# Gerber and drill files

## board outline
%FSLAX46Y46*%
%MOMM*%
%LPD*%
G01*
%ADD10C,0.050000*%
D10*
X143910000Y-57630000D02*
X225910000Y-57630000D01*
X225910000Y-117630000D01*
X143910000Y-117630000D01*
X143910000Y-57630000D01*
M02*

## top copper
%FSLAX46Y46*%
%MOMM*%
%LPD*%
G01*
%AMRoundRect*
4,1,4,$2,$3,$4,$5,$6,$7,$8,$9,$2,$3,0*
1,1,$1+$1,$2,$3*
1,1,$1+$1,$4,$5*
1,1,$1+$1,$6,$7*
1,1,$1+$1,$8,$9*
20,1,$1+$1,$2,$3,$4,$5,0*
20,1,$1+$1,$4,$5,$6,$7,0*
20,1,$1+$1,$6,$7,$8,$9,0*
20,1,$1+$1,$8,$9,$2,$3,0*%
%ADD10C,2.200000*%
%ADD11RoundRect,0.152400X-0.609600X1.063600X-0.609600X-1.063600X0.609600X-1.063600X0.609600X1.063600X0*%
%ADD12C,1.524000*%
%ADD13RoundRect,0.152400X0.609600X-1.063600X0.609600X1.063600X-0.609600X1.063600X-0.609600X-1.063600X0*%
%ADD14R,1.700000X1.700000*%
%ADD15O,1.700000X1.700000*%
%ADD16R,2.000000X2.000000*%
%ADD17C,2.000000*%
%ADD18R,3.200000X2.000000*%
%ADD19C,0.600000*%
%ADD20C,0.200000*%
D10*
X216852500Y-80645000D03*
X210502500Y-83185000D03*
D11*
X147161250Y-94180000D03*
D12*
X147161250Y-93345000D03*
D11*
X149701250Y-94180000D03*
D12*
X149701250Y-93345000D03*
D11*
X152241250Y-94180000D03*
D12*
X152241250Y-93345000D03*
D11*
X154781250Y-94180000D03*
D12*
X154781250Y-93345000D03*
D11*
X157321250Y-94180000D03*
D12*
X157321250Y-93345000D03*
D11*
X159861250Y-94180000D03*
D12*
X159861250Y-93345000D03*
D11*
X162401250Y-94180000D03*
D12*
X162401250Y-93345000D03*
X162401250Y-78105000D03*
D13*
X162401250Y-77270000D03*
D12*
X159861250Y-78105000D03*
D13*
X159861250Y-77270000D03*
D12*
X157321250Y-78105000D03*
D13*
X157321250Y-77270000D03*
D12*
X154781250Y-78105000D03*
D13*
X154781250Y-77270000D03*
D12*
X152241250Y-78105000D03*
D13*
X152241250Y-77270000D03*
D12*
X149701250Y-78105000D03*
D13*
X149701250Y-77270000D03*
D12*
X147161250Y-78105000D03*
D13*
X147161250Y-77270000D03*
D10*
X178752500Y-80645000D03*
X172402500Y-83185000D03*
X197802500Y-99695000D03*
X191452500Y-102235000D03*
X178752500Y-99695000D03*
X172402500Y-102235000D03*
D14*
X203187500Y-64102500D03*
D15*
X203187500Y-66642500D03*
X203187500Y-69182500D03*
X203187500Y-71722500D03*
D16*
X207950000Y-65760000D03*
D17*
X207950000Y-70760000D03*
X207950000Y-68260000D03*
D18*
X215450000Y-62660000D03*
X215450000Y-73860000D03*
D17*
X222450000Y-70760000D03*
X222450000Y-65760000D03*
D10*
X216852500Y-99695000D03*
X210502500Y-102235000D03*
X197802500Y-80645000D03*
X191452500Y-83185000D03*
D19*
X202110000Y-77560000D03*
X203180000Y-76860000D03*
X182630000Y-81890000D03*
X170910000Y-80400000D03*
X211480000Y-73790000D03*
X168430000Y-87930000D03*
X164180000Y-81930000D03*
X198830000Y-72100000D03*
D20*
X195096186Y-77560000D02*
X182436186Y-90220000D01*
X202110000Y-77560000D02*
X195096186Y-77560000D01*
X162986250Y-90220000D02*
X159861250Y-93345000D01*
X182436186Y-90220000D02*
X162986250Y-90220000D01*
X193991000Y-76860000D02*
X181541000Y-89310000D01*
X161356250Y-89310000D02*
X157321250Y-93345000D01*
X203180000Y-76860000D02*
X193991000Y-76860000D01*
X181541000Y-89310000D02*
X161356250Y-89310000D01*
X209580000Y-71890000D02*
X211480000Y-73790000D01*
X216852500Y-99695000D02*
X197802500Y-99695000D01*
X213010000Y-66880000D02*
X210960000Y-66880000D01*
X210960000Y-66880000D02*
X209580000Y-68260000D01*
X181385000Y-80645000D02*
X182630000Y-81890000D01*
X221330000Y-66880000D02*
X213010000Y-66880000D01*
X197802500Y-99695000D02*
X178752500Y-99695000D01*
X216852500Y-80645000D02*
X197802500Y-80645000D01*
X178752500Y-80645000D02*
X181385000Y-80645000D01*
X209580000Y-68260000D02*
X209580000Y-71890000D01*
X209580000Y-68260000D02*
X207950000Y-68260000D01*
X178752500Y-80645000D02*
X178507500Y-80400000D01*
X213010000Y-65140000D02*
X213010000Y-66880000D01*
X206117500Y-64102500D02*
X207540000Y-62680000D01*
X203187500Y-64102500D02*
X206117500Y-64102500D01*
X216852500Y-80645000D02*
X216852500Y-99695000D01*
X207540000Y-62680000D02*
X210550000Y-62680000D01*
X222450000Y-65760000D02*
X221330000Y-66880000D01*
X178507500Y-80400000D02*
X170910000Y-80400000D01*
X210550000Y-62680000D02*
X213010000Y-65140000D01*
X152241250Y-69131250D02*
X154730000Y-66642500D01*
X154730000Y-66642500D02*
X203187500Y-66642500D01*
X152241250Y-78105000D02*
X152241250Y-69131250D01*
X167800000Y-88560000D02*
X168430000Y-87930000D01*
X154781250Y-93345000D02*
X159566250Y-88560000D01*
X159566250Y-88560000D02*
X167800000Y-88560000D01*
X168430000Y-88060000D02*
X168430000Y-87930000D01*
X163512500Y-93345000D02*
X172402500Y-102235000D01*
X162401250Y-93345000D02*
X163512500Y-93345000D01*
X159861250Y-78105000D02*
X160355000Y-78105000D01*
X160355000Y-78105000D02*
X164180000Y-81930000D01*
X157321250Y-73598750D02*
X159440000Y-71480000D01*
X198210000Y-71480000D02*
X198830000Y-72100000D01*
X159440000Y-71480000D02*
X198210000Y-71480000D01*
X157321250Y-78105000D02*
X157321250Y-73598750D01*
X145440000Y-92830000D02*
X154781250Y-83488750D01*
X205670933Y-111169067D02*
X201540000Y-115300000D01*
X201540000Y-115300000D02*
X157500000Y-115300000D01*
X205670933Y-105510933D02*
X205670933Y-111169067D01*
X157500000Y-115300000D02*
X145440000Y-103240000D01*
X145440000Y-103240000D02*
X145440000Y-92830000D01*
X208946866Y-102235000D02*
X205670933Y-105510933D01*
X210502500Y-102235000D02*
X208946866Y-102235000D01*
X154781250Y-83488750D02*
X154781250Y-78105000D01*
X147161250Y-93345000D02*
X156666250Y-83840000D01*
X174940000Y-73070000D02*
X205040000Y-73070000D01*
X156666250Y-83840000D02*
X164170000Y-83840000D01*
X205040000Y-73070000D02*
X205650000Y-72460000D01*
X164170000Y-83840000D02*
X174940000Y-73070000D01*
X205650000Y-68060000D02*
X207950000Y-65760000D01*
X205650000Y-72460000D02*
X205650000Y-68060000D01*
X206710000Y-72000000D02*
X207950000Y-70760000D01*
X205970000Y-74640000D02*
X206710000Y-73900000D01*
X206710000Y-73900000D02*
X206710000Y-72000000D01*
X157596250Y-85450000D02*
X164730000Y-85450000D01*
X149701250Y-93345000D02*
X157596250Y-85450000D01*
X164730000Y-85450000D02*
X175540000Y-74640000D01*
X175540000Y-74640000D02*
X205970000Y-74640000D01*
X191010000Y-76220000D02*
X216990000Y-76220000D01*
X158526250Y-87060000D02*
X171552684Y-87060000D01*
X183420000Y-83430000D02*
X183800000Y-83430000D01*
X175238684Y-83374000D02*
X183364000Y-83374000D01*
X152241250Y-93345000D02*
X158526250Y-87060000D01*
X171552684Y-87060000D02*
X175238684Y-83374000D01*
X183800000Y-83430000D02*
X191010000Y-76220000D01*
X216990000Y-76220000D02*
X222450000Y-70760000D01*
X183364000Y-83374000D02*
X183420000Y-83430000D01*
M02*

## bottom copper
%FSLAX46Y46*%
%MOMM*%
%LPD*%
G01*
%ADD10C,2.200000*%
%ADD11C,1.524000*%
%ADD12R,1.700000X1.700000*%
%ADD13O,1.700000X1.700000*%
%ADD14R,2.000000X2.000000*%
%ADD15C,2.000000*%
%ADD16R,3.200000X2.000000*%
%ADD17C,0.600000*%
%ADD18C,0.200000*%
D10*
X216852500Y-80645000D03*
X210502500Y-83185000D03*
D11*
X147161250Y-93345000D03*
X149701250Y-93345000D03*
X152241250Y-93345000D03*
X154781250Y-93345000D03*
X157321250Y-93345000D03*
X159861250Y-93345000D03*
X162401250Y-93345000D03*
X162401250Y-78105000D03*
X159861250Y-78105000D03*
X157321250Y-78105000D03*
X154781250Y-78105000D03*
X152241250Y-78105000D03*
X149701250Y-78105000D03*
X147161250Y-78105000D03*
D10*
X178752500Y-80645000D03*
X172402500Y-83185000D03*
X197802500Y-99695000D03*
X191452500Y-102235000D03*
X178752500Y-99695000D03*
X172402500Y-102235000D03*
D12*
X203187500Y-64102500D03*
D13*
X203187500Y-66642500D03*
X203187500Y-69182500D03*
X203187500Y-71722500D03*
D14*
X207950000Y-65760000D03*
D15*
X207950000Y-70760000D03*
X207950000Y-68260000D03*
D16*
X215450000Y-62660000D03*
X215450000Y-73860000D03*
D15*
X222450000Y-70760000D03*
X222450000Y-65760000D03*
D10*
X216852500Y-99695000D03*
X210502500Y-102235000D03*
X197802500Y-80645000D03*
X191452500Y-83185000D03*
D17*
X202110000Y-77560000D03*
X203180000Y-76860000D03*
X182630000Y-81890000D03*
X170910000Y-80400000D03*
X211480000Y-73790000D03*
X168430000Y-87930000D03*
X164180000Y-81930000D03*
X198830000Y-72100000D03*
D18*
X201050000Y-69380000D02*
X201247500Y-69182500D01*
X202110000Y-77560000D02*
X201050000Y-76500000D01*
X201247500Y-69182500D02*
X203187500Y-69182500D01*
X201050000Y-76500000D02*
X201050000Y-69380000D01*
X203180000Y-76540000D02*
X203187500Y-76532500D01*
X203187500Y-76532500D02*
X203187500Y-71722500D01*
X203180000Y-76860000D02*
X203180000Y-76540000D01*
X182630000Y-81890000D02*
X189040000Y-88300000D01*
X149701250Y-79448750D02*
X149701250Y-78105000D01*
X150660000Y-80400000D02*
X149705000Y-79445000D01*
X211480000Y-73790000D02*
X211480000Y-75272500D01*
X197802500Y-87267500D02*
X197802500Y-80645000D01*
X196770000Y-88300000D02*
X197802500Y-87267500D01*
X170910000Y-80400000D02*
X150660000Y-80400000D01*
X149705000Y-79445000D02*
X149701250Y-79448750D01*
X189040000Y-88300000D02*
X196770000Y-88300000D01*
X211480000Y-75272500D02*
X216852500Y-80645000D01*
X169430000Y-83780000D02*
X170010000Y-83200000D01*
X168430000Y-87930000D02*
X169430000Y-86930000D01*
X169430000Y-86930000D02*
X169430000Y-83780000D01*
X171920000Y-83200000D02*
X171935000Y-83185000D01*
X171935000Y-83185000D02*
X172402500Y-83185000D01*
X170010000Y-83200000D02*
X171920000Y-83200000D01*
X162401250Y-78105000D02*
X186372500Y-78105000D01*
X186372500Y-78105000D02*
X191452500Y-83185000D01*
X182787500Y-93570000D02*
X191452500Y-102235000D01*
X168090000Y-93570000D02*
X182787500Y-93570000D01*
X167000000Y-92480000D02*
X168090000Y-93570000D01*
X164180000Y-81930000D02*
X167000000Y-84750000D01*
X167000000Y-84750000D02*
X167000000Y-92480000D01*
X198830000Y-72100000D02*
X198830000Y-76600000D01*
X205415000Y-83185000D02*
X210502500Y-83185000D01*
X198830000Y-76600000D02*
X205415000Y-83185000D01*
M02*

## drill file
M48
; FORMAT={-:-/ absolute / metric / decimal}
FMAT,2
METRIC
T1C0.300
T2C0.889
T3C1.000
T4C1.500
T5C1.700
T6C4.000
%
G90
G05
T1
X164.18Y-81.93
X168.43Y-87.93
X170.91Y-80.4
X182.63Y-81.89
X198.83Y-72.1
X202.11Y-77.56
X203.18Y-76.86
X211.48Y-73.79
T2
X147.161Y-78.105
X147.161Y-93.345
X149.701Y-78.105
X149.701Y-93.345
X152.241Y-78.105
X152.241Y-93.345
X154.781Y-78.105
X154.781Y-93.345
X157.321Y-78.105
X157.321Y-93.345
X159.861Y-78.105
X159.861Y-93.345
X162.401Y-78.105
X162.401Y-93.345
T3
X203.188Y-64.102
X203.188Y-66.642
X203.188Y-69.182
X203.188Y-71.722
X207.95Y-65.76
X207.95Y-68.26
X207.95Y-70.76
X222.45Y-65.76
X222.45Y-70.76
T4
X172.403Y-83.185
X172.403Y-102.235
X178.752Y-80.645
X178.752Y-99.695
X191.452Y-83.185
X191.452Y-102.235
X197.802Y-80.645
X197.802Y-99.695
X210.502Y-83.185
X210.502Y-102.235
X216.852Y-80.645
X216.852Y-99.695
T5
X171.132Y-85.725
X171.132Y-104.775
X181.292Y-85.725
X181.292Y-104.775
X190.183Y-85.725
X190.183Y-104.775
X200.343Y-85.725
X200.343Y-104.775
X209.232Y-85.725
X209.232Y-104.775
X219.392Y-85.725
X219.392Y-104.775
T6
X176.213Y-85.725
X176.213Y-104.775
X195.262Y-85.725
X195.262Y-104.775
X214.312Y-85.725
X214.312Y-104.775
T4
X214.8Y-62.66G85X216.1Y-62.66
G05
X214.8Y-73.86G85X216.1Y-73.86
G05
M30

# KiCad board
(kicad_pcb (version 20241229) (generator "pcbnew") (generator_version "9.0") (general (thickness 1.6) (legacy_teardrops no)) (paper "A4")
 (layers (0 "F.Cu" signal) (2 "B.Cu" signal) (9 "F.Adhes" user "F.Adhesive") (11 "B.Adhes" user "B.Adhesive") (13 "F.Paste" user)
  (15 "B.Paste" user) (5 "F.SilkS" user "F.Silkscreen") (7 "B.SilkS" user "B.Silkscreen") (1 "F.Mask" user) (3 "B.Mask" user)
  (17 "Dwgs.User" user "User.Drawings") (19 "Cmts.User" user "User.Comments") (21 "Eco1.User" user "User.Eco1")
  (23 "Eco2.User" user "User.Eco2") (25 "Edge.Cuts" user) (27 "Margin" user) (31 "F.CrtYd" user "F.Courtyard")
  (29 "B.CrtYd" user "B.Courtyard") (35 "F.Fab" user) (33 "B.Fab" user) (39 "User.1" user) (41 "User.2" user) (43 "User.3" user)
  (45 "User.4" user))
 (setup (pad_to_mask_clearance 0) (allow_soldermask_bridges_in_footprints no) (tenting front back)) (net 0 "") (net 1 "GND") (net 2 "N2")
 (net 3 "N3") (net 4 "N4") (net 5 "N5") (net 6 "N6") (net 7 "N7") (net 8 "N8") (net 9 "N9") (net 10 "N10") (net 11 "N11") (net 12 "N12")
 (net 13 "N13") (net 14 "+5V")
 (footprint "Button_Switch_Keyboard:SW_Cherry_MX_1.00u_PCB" (layer "F.Cu") (at 216.8525 80.645)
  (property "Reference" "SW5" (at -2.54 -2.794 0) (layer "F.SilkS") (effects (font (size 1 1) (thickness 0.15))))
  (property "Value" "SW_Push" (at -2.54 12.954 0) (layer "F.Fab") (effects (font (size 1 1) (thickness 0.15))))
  (pad "" np_thru_hole circle (at -7.62 5.08) (size 1.7 1.7) (drill 1.7) (layers "*.Cu" "*.Mask"))
  (pad "" np_thru_hole circle (at -2.54 5.08) (size 4 4) (drill 4) (layers "*.Cu" "*.Mask"))
  (pad "" np_thru_hole circle (at 2.54 5.08) (size 1.7 1.7) (drill 1.7) (layers "*.Cu" "*.Mask"))
  (pad "1" thru_hole circle (at 0 0) (size 2.2 2.2) (drill 1.5) (layers "*.Cu" "*.Mask") (remove_unused_layers no) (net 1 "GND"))
  (pad "2" thru_hole circle (at -6.35 2.54) (size 2.2 2.2) (drill 1.5) (layers "*.Cu" "*.Mask") (remove_unused_layers no) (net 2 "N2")))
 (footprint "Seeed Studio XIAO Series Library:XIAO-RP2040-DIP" (layer "F.Cu") (at 154.78125 85.725 90)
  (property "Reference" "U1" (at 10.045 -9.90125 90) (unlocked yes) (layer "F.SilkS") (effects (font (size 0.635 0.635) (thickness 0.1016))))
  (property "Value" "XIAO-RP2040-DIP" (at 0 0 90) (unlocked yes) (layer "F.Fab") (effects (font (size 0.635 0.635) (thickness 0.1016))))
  (pad "1" smd roundrect (at -8.455 -7.62 270) (size 2.432 1.524) (layers "F.Cu" "F.Mask") (roundrect_rratio 0.1) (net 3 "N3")
   (thermal_bridge_angle 45))
  (pad "1" thru_hole circle (at -7.62 -7.62 270) (size 1.524 1.524) (drill 0.889) (layers "*.Cu" "*.Mask") (remove_unused_layers no)
   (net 3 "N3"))
  (pad "2" smd roundrect (at -8.455 -5.08 270) (size 2.432 1.524) (layers "F.Cu" "F.Mask") (roundrect_rratio 0.1) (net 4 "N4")
   (thermal_bridge_angle 45))
  (pad "2" thru_hole circle (at -7.62 -5.08 270) (size 1.524 1.524) (drill 0.889) (layers "*.Cu" "*.Mask") (remove_unused_layers no)
   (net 4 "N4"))
  (pad "3" smd roundrect (at -8.455 -2.54 270) (size 2.432 1.524) (layers "F.Cu" "F.Mask") (roundrect_rratio 0.1) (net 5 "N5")
   (thermal_bridge_angle 45))
  (pad "3" thru_hole circle (at -7.62 -2.54 270) (size 1.524 1.524) (drill 0.889) (layers "*.Cu" "*.Mask") (remove_unused_layers no)
   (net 5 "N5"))
  (pad "4" smd roundrect (at -8.455 0 270) (size 2.432 1.524) (layers "F.Cu" "F.Mask") (roundrect_rratio 0.1) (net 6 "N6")
   (thermal_bridge_angle 45))
  (pad "4" thru_hole circle (at -7.62 0 270) (size 1.524 1.524) (drill 0.889) (layers "*.Cu" "*.Mask") (remove_unused_layers no)
   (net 6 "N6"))
  (pad "5" smd roundrect (at -8.455 2.54 270) (size 2.432 1.524) (layers "F.Cu" "F.Mask") (roundrect_rratio 0.1) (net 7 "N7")
   (thermal_bridge_angle 45))
  (pad "5" thru_hole circle (at -7.62 2.54 270) (size 1.524 1.524) (drill 0.889) (layers "*.Cu" "*.Mask") (remove_unused_layers no)
   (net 7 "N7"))
  (pad "6" smd roundrect (at -8.455 5.08 270) (size 2.432 1.524) (layers "F.Cu" "F.Mask") (roundrect_rratio 0.1) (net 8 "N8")
   (thermal_bridge_angle 45))
  (pad "6" thru_hole circle (at -7.62 5.08 270) (size 1.524 1.524) (drill 0.889) (layers "*.Cu" "*.Mask") (remove_unused_layers no)
   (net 8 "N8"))
  (pad "7" smd roundrect (at -8.455 7.62 270) (size 2.432 1.524) (layers "F.Cu" "F.Mask") (roundrect_rratio 0.1) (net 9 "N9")
   (thermal_bridge_angle 45))
  (pad "7" thru_hole circle (at -7.62 7.62 270) (size 1.524 1.524) (drill 0.889) (layers "*.Cu" "*.Mask") (remove_unused_layers no)
   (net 9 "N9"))
  (pad "8" thru_hole circle (at 7.62 7.62 90) (size 1.524 1.524) (drill 0.889) (layers "*.Cu" "*.Mask") (remove_unused_layers no)
   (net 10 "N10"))
  (pad "8" smd roundrect (at 8.455 7.62 90) (size 2.432 1.524) (layers "F.Cu" "F.Mask") (roundrect_rratio 0.1) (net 10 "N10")
   (thermal_bridge_angle 45))
  (pad "9" thru_hole circle (at 7.62 5.08 90) (size 1.524 1.524) (drill 0.889) (layers "*.Cu" "*.Mask") (remove_unused_layers no)
   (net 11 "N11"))
  (pad "9" smd roundrect (at 8.455 5.08 90) (size 2.432 1.524) (layers "F.Cu" "F.Mask") (roundrect_rratio 0.1) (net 11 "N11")
   (thermal_bridge_angle 45))
  (pad "10" thru_hole circle (at 7.62 2.54 90) (size 1.524 1.524) (drill 0.889) (layers "*.Cu" "*.Mask") (remove_unused_layers no)
   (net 2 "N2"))
  (pad "10" smd roundrect (at 8.455 2.54 90) (size 2.432 1.524) (layers "F.Cu" "F.Mask") (roundrect_rratio 0.1) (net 2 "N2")
   (thermal_bridge_angle 45))
  (pad "11" thru_hole circle (at 7.62 0 90) (size 1.524 1.524) (drill 0.889) (layers "*.Cu" "*.Mask") (remove_unused_layers no)
   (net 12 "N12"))
  (pad "11" smd roundrect (at 8.455 0 90) (size 2.432 1.524) (layers "F.Cu" "F.Mask") (roundrect_rratio 0.1) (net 12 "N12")
   (thermal_bridge_angle 45))
  (pad "12" thru_hole circle (at 7.62 -2.54 90) (size 1.524 1.524) (drill 0.889) (layers "*.Cu" "*.Mask") (remove_unused_layers no)
   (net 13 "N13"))
  (pad "12" smd roundrect (at 8.455 -2.54 90) (size 2.432 1.524) (layers "F.Cu" "F.Mask") (roundrect_rratio 0.1) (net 13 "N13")
   (thermal_bridge_angle 45))
  (pad "13" thru_hole circle (at 7.62 -5.08 90) (size 1.524 1.524) (drill 0.889) (layers "*.Cu" "*.Mask") (remove_unused_layers no)
   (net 1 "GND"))
  (pad "13" smd roundrect (at 8.455 -5.08 90) (size 2.432 1.524) (layers "F.Cu" "F.Mask") (roundrect_rratio 0.1) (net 1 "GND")
   (thermal_bridge_angle 45))
  (pad "14" thru_hole circle (at 7.62 -7.62 90) (size 1.524 1.524) (drill 0.889) (layers "*.Cu" "*.Mask") (remove_unused_layers no)
   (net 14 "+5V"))
  (pad "14" smd roundrect (at 8.455 -7.62 90) (size 2.432 1.524) (layers "F.Cu" "F.Mask") (roundrect_rratio 0.1) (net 14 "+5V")
   (thermal_bridge_angle 45)))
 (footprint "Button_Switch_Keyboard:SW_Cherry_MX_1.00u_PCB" (layer "F.Cu") (at 178.7525 80.645)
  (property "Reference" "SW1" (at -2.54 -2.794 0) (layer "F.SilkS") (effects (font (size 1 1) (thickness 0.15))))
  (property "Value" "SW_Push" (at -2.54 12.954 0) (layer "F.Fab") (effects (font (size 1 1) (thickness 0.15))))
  (pad "" np_thru_hole circle (at -7.62 5.08) (size 1.7 1.7) (drill 1.7) (layers "*.Cu" "*.Mask"))
  (pad "" np_thru_hole circle (at -2.54 5.08) (size 4 4) (drill 4) (layers "*.Cu" "*.Mask"))
  (pad "" np_thru_hole circle (at 2.54 5.08) (size 1.7 1.7) (drill 1.7) (layers "*.Cu" "*.Mask"))
  (pad "1" thru_hole circle (at 0 0) (size 2.2 2.2) (drill 1.5) (layers "*.Cu" "*.Mask") (remove_unused_layers no) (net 1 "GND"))
  (pad "2" thru_hole circle (at -6.35 2.54) (size 2.2 2.2) (drill 1.5) (layers "*.Cu" "*.Mask") (remove_unused_layers no) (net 6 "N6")))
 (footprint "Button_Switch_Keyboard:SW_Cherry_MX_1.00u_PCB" (layer "F.Cu") (at 197.8025 99.695)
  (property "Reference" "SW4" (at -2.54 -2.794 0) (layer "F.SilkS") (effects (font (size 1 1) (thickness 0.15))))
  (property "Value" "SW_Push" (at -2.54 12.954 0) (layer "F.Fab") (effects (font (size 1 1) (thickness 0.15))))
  (pad "" np_thru_hole circle (at -7.62 5.08) (size 1.7 1.7) (drill 1.7) (layers "*.Cu" "*.Mask"))
  (pad "" np_thru_hole circle (at -2.54 5.08) (size 4 4) (drill 4) (layers "*.Cu" "*.Mask"))
  (pad "" np_thru_hole circle (at 2.54 5.08) (size 1.7 1.7) (drill 1.7) (layers "*.Cu" "*.Mask"))
  (pad "1" thru_hole circle (at 0 0) (size 2.2 2.2) (drill 1.5) (layers "*.Cu" "*.Mask") (remove_unused_layers no) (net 1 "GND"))
  (pad "2" thru_hole circle (at -6.35 2.54) (size 2.2 2.2) (drill 1.5) (layers "*.Cu" "*.Mask") (remove_unused_layers no) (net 11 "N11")))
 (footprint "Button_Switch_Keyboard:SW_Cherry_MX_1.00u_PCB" (layer "F.Cu") (at 178.7525 99.695)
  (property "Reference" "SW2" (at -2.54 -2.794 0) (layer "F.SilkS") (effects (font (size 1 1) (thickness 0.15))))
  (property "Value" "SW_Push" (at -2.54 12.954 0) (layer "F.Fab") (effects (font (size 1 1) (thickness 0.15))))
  (pad "" np_thru_hole circle (at -7.62 5.08) (size 1.7 1.7) (drill 1.7) (layers "*.Cu" "*.Mask"))
  (pad "" np_thru_hole circle (at -2.54 5.08) (size 4 4) (drill 4) (layers "*.Cu" "*.Mask"))
  (pad "" np_thru_hole circle (at 2.54 5.08) (size 1.7 1.7) (drill 1.7) (layers "*.Cu" "*.Mask"))
  (pad "1" thru_hole circle (at 0 0) (size 2.2 2.2) (drill 1.5) (layers "*.Cu" "*.Mask") (remove_unused_layers no) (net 1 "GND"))
  (pad "2" thru_hole circle (at -6.35 2.54) (size 2.2 2.2) (drill 1.5) (layers "*.Cu" "*.Mask") (remove_unused_layers no) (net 9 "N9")))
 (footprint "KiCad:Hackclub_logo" (layer "F.Cu") (at 156.223071 67.360382)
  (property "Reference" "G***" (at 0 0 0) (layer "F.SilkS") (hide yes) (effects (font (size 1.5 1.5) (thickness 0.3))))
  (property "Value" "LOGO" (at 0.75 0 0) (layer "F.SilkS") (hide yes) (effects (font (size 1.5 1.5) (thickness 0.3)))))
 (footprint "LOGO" (layer "F.Cu") (at 155.84 108.43)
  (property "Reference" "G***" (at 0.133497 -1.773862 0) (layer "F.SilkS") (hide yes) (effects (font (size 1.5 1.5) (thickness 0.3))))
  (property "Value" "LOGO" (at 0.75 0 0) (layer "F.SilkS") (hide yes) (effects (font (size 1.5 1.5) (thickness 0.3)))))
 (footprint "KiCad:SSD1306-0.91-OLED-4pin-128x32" (layer "F.Cu") (at 166.6875 61.9125)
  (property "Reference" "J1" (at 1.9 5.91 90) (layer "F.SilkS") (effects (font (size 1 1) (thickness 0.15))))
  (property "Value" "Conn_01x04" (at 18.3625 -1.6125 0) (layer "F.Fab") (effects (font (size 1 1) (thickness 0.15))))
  (pad "1" thru_hole rect (at 36.5 2.19) (size 1.7 1.7) (drill 1) (layers "*.Cu" "*.Mask") (remove_unused_layers no) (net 1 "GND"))
  (pad "2" thru_hole oval (at 36.5 4.73) (size 1.7 1.7) (drill 1) (layers "*.Cu" "*.Mask") (remove_unused_layers no) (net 13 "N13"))
  (pad "3" thru_hole oval (at 36.5 7.27) (size 1.7 1.7) (drill 1) (layers "*.Cu" "*.Mask") (remove_unused_layers no) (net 8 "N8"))
  (pad "4" thru_hole oval (at 36.5 9.81) (size 1.7 1.7) (drill 1) (layers "*.Cu" "*.Mask") (remove_unused_layers no) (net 7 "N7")))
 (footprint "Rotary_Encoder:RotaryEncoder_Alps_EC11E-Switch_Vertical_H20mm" (layer "F.Cu") (at 207.95 65.76)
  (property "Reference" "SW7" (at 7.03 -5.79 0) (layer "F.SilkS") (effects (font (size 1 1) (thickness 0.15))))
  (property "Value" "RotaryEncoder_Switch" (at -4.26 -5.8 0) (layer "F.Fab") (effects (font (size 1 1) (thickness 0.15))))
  (pad "A" thru_hole rect (at 0 0) (size 2 2) (drill 1) (layers "*.Cu" "*.Mask") (remove_unused_layers no) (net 3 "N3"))
  (pad "B" thru_hole circle (at 0 5) (size 2 2) (drill 1) (layers "*.Cu" "*.Mask") (remove_unused_layers no) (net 4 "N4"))
  (pad "C" thru_hole circle (at 0 2.5) (size 2 2) (drill 1) (layers "*.Cu" "*.Mask") (remove_unused_layers no) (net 1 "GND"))
  (pad "MP" thru_hole rect (at 7.5 -3.1) (size 3.2 2) (drill oval 2.8 1.5) (layers "*.Cu" "*.Mask") (remove_unused_layers no))
  (pad "MP" thru_hole rect (at 7.5 8.1) (size 3.2 2) (drill oval 2.8 1.5) (layers "*.Cu" "*.Mask") (remove_unused_layers no))
  (pad "S1" thru_hole circle (at 14.5 5) (size 2 2) (drill 1) (layers "*.Cu" "*.Mask") (remove_unused_layers no) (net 5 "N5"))
  (pad "S2" thru_hole circle (at 14.5 0) (size 2 2) (drill 1) (layers "*.Cu" "*.Mask") (remove_unused_layers no) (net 1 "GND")))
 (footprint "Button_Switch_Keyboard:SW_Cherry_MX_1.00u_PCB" (layer "F.Cu") (at 216.8525 99.695)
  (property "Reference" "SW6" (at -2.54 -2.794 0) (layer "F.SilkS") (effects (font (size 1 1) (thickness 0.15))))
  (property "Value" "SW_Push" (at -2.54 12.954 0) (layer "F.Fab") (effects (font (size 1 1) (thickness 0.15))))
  (pad "" np_thru_hole circle (at -7.62 5.08) (size 1.7 1.7) (drill 1.7) (layers "*.Cu" "*.Mask"))
  (pad "" np_thru_hole circle (at -2.54 5.08) (size 4 4) (drill 4) (layers "*.Cu" "*.Mask"))
  (pad "" np_thru_hole circle (at 2.54 5.08) (size 1.7 1.7) (drill 1.7) (layers "*.Cu" "*.Mask"))
  (pad "1" thru_hole circle (at 0 0) (size 2.2 2.2) (drill 1.5) (layers "*.Cu" "*.Mask") (remove_unused_layers no) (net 1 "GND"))
  (pad "2" thru_hole circle (at -6.35 2.54) (size 2.2 2.2) (drill 1.5) (layers "*.Cu" "*.Mask") (remove_unused_layers no) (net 12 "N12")))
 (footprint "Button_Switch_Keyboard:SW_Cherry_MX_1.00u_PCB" (layer "F.Cu") (at 197.8025 80.645)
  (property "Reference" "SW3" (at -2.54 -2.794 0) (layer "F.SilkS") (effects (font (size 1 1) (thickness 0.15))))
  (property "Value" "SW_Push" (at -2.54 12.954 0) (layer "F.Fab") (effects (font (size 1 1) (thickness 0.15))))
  (pad "" np_thru_hole circle (at -7.62 5.08) (size 1.7 1.7) (drill 1.7) (layers "*.Cu" "*.Mask"))
  (pad "" np_thru_hole circle (at -2.54 5.08) (size 4 4) (drill 4) (layers "*.Cu" "*.Mask"))
  (pad "" np_thru_hole circle (at 2.54 5.08) (size 1.7 1.7) (drill 1.7) (layers "*.Cu" "*.Mask"))
  (pad "1" thru_hole circle (at 0 0) (size 2.2 2.2) (drill 1.5) (layers "*.Cu" "*.Mask") (remove_unused_layers no) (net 1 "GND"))
  (pad "2" thru_hole circle (at -6.35 2.54) (size 2.2 2.2) (drill 1.5) (layers "*.Cu" "*.Mask") (remove_unused_layers no) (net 10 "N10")))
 (gr_rect (start 143.91 57.63) (end 225.91 117.63) (stroke (width 0.05) (type solid)) (fill no) (layer "Edge.Cuts"))
 (segment (start 195.096186 77.56) (end 182.436186 90.22) (width 0.2) (layer "F.Cu") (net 8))
 (segment (start 202.11 77.56) (end 195.096186 77.56) (width 0.2) (layer "F.Cu") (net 8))
 (segment (start 162.98625 90.22) (end 159.86125 93.345) (width 0.2) (layer "F.Cu") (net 8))
 (segment (start 182.436186 90.22) (end 162.98625 90.22) (width 0.2) (layer "F.Cu") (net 8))
 (via (at 202.11 77.56) (size 0.6) (drill 0.3) (layers "F.Cu" "B.Cu") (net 8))
 (segment (start 201.05 69.38) (end 201.2475 69.1825) (width 0.2) (layer "B.Cu") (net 8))
 (segment (start 202.11 77.56) (end 201.05 76.5) (width 0.2) (layer "B.Cu") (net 8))
 (segment (start 201.2475 69.1825) (end 203.1875 69.1825) (width 0.2) (layer "B.Cu") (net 8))
 (segment (start 201.05 76.5) (end 201.05 69.38) (width 0.2) (layer "B.Cu") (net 8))
 (segment (start 193.991 76.86) (end 181.541 89.31) (width 0.2) (layer "F.Cu") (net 7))
 (segment (start 161.35625 89.31) (end 157.32125 93.345) (width 0.2) (layer "F.Cu") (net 7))
 (segment (start 203.18 76.86) (end 193.991 76.86) (width 0.2) (layer "F.Cu") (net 7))
 (segment (start 181.541 89.31) (end 161.35625 89.31) (width 0.2) (layer "F.Cu") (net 7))
 (via (at 203.18 76.86) (size 0.6) (drill 0.3) (layers "F.Cu" "B.Cu") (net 7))
 (segment (start 203.18 76.54) (end 203.1875 76.5325) (width 0.2) (layer "B.Cu") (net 7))
 (segment (start 203.1875 76.5325) (end 203.1875 71.7225) (width 0.2) (layer "B.Cu") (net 7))
 (segment (start 203.18 76.86) (end 203.18 76.54) (width 0.2) (layer "B.Cu") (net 7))
 (segment (start 209.58 71.89) (end 211.48 73.79) (width 0.2) (layer "F.Cu") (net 1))
 (segment (start 216.8525 99.695) (end 197.8025 99.695) (width 0.2) (layer "F.Cu") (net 1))
 (segment (start 213.01 66.88) (end 210.96 66.88) (width 0.2) (layer "F.Cu") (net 1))
 (segment (start 210.96 66.88) (end 209.58 68.26) (width 0.2) (layer "F.Cu") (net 1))
 (segment (start 181.385 80.645) (end 182.63 81.89) (width 0.2) (layer "F.Cu") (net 1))
 (segment (start 221.33 66.88) (end 213.01 66.88) (width 0.2) (layer "F.Cu") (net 1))
 (segment (start 197.8025 99.695) (end 178.7525 99.695) (width 0.2) (layer "F.Cu") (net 1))
 (segment (start 216.8525 80.645) (end 197.8025 80.645) (width 0.2) (layer "F.Cu") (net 1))
 (segment (start 178.7525 80.645) (end 181.385 80.645) (width 0.2) (layer "F.Cu") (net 1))
 (segment (start 209.58 68.26) (end 209.58 71.89) (width 0.2) (layer "F.Cu") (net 1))
 (segment (start 209.58 68.26) (end 207.95 68.26) (width 0.2) (layer "F.Cu") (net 1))
 (segment (start 178.7525 80.645) (end 178.5075 80.4) (width 0.2) (layer "F.Cu") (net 1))
 (segment (start 213.01 65.14) (end 213.01 66.88) (width 0.2) (layer "F.Cu") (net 1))
 (segment (start 206.1175 64.1025) (end 207.54 62.68) (width 0.2) (layer "F.Cu") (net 1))
 (segment (start 203.1875 64.1025) (end 206.1175 64.1025) (width 0.2) (layer "F.Cu") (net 1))
 (segment (start 216.8525 80.645) (end 216.8525 99.695) (width 0.2) (layer "F.Cu") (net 1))
 (segment (start 207.54 62.68) (end 210.55 62.68) (width 0.2) (layer "F.Cu") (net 1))
 (segment (start 222.45 65.76) (end 221.33 66.88) (width 0.2) (layer "F.Cu") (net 1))
 (segment (start 178.5075 80.4) (end 170.91 80.4) (width 0.2) (layer "F.Cu") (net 1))
 (segment (start 210.55 62.68) (end 213.01 65.14) (width 0.2) (layer "F.Cu") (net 1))
 (via (at 182.63 81.89) (size 0.6) (drill 0.3) (layers "F.Cu" "B.Cu") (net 1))
 (via (at 170.91 80.4) (size 0.6) (drill 0.3) (layers "F.Cu" "B.Cu") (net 1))
 (via (at 211.48 73.79) (size 0.6) (drill 0.3) (layers "F.Cu" "B.Cu") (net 1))
 (segment (start 182.63 81.89) (end 189.04 88.3) (width 0.2) (layer "B.Cu") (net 1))
 (segment (start 149.70125 79.44875) (end 149.70125 78.105) (width 0.2) (layer "B.Cu") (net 1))
 (segment (start 150.66 80.4) (end 149.705 79.445) (width 0.2) (layer "B.Cu") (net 1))
 (segment (start 211.48 73.79) (end 211.48 75.2725) (width 0.2) (layer "B.Cu") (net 1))
 (segment (start 197.8025 87.2675) (end 197.8025 80.645) (width 0.2) (layer "B.Cu") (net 1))
 (segment (start 196.77 88.3) (end 197.8025 87.2675) (width 0.2) (layer "B.Cu") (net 1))
 (segment (start 170.91 80.4) (end 150.66 80.4) (width 0.2) (layer "B.Cu") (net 1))
 (segment (start 149.705 79.445) (end 149.70125 79.44875) (width 0.2) (layer "B.Cu") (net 1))
 (segment (start 189.04 88.3) (end 196.77 88.3) (width 0.2) (layer "B.Cu") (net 1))
 (segment (start 211.48 75.2725) (end 216.8525 80.645) (width 0.2) (layer "B.Cu") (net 1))
 (segment (start 152.24125 69.13125) (end 154.73 66.6425) (width 0.2) (layer "F.Cu") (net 13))
 (segment (start 154.73 66.6425) (end 203.1875 66.6425) (width 0.2) (layer "F.Cu") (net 13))
 (segment (start 152.24125 78.105) (end 152.24125 69.13125) (width 0.2) (layer "F.Cu") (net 13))
 (segment (start 167.8 88.56) (end 168.43 87.93) (width 0.2) (layer "F.Cu") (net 6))
 (segment (start 154.78125 93.345) (end 159.56625 88.56) (width 0.2) (layer "F.Cu") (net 6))
 (segment (start 159.56625 88.56) (end 167.8 88.56) (width 0.2) (layer "F.Cu") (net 6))
 (segment (start 168.43 88.06) (end 168.43 87.93) (width 0.2) (layer "F.Cu") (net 6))
 (via (at 168.43 87.93) (size 0.6) (drill 0.3) (layers "F.Cu" "B.Cu") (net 6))
 (segment (start 169.43 83.78) (end 170.01 83.2) (width 0.2) (layer "B.Cu") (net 6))
 (segment (start 168.43 87.93) (end 169.43 86.93) (width 0.2) (layer "B.Cu") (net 6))
 (segment (start 169.43 86.93) (end 169.43 83.78) (width 0.2) (layer "B.Cu") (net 6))
 (segment (start 171.92 83.2) (end 171.935 83.185) (width 0.2) (layer "B.Cu") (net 6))
 (segment (start 171.935 83.185) (end 172.4025 83.185) (width 0.2) (layer "B.Cu") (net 6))
 (segment (start 170.01 83.2) (end 171.92 83.2) (width 0.2) (layer "B.Cu") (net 6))
 (segment (start 163.5125 93.345) (end 172.4025 102.235) (width 0.2) (layer "F.Cu") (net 9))
 (segment (start 162.40125 93.345) (end 163.5125 93.345) (width 0.2) (layer "F.Cu") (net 9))
 (segment (start 162.40125 78.105) (end 186.3725 78.105) (width 0.2) (layer "B.Cu") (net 10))
 (segment (start 186.3725 78.105) (end 191.4525 83.185) (width 0.2) (layer "B.Cu") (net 10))
 (segment (start 159.86125 78.105) (end 160.355 78.105) (width 0.2) (layer "F.Cu") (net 11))
 (segment (start 160.355 78.105) (end 164.18 81.93) (width 0.2) (layer "F.Cu") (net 11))
 (via (at 164.18 81.93) (size 0.6) (drill 0.3) (layers "F.Cu" "B.Cu") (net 11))
 (segment (start 182.7875 93.57) (end 191.4525 102.235) (width 0.2) (layer "B.Cu") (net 11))
 (segment (start 168.09 93.57) (end 182.7875 93.57) (width 0.2) (layer "B.Cu") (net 11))
 (segment (start 167 92.48) (end 168.09 93.57) (width 0.2) (layer "B.Cu") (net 11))
 (segment (start 164.18 81.93) (end 167 84.75) (width 0.2) (layer "B.Cu") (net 11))
 (segment (start 167 84.75) (end 167 92.48) (width 0.2) (layer "B.Cu") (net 11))
 (segment (start 157.32125 73.59875) (end 159.44 71.48) (width 0.2) (layer "F.Cu") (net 2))
 (segment (start 198.21 71.48) (end 198.83 72.1) (width 0.2) (layer "F.Cu") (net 2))
 (segment (start 159.44 71.48) (end 198.21 71.48) (width 0.2) (layer "F.Cu") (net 2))
 (segment (start 157.32125 78.105) (end 157.32125 73.59875) (width 0.2) (layer "F.Cu") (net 2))
 (via (at 198.83 72.1) (size 0.6) (drill 0.3) (layers "F.Cu" "B.Cu") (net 2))
 (segment (start 198.83 72.1) (end 198.83 76.6) (width 0.2) (layer "B.Cu") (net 2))
 (segment (start 205.415 83.185) (end 210.5025 83.185) (width 0.2) (layer "B.Cu") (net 2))
 (segment (start 198.83 76.6) (end 205.415 83.185) (width 0.2) (layer "B.Cu") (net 2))
 (segment (start 145.44 92.83) (end 154.78125 83.48875) (width 0.2) (layer "F.Cu") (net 12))
 (segment (start 205.670933 111.169067) (end 201.54 115.3) (width 0.2) (layer "F.Cu") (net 12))
 (segment (start 201.54 115.3) (end 157.5 115.3) (width 0.2) (layer "F.Cu") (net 12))
 (segment (start 205.670933 105.510933) (end 205.670933 111.169067) (width 0.2) (layer "F.Cu") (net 12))
 (segment (start 157.5 115.3) (end 145.44 103.24) (width 0.2) (layer "F.Cu") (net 12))
 (segment (start 145.44 103.24) (end 145.44 92.83) (width 0.2) (layer "F.Cu") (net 12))
 (segment (start 208.946866 102.235) (end 205.670933 105.510933) (width 0.2) (layer "F.Cu") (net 12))
 (segment (start 210.5025 102.235) (end 208.946866 102.235) (width 0.2) (layer "F.Cu") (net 12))
 (segment (start 154.78125 83.48875) (end 154.78125 78.105) (width 0.2) (layer "F.Cu") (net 12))
 (segment (start 147.16125 93.345) (end 156.66625 83.84) (width 0.2) (layer "F.Cu") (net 3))
 (segment (start 174.94 73.07) (end 205.04 73.07) (width 0.2) (layer "F.Cu") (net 3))
 (segment (start 156.66625 83.84) (end 164.17 83.84) (width 0.2) (layer "F.Cu") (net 3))
 (segment (start 205.04 73.07) (end 205.65 72.46) (width 0.2) (layer "F.Cu") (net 3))
 (segment (start 164.17 83.84) (end 174.94 73.07) (width 0.2) (layer "F.Cu") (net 3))
 (segment (start 205.65 68.06) (end 207.95 65.76) (width 0.2) (layer "F.Cu") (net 3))
 (segment (start 205.65 72.46) (end 205.65 68.06) (width 0.2) (layer "F.Cu") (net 3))
 (segment (start 206.71 72) (end 207.95 70.76) (width 0.2) (layer "F.Cu") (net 4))
 (segment (start 205.97 74.64) (end 206.71 73.9) (width 0.2) (layer "F.Cu") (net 4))
 (segment (start 206.71 73.9) (end 206.71 72) (width 0.2) (layer "F.Cu") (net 4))
 (segment (start 157.59625 85.45) (end 164.73 85.45) (width 0.2) (layer "F.Cu") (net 4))
 (segment (start 149.70125 93.345) (end 157.59625 85.45) (width 0.2) (layer "F.Cu") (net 4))
 (segment (start 164.73 85.45) (end 175.54 74.64) (width 0.2) (layer "F.Cu") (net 4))
 (segment (start 175.54 74.64) (end 205.97 74.64) (width 0.2) (layer "F.Cu") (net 4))
 (segment (start 191.01 76.22) (end 216.99 76.22) (width 0.2) (layer "F.Cu") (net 5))
 (segment (start 158.52625 87.06) (end 171.552684 87.06) (width 0.2) (layer "F.Cu") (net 5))
 (segment (start 183.42 83.43) (end 183.8 83.43) (width 0.2) (layer "F.Cu") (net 5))
 (segment (start 175.238684 83.374) (end 183.364 83.374) (width 0.2) (layer "F.Cu") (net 5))
 (segment (start 152.24125 93.345) (end 158.52625 87.06) (width 0.2) (layer "F.Cu") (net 5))
 (segment (start 171.552684 87.06) (end 175.238684 83.374) (width 0.2) (layer "F.Cu") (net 5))
 (segment (start 183.8 83.43) (end 191.01 76.22) (width 0.2) (layer "F.Cu") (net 5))
 (segment (start 216.99 76.22) (end 222.45 70.76) (width 0.2) (layer "F.Cu") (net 5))
 (segment (start 183.364 83.374) (end 183.42 83.43) (width 0.2) (layer "F.Cu") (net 5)))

